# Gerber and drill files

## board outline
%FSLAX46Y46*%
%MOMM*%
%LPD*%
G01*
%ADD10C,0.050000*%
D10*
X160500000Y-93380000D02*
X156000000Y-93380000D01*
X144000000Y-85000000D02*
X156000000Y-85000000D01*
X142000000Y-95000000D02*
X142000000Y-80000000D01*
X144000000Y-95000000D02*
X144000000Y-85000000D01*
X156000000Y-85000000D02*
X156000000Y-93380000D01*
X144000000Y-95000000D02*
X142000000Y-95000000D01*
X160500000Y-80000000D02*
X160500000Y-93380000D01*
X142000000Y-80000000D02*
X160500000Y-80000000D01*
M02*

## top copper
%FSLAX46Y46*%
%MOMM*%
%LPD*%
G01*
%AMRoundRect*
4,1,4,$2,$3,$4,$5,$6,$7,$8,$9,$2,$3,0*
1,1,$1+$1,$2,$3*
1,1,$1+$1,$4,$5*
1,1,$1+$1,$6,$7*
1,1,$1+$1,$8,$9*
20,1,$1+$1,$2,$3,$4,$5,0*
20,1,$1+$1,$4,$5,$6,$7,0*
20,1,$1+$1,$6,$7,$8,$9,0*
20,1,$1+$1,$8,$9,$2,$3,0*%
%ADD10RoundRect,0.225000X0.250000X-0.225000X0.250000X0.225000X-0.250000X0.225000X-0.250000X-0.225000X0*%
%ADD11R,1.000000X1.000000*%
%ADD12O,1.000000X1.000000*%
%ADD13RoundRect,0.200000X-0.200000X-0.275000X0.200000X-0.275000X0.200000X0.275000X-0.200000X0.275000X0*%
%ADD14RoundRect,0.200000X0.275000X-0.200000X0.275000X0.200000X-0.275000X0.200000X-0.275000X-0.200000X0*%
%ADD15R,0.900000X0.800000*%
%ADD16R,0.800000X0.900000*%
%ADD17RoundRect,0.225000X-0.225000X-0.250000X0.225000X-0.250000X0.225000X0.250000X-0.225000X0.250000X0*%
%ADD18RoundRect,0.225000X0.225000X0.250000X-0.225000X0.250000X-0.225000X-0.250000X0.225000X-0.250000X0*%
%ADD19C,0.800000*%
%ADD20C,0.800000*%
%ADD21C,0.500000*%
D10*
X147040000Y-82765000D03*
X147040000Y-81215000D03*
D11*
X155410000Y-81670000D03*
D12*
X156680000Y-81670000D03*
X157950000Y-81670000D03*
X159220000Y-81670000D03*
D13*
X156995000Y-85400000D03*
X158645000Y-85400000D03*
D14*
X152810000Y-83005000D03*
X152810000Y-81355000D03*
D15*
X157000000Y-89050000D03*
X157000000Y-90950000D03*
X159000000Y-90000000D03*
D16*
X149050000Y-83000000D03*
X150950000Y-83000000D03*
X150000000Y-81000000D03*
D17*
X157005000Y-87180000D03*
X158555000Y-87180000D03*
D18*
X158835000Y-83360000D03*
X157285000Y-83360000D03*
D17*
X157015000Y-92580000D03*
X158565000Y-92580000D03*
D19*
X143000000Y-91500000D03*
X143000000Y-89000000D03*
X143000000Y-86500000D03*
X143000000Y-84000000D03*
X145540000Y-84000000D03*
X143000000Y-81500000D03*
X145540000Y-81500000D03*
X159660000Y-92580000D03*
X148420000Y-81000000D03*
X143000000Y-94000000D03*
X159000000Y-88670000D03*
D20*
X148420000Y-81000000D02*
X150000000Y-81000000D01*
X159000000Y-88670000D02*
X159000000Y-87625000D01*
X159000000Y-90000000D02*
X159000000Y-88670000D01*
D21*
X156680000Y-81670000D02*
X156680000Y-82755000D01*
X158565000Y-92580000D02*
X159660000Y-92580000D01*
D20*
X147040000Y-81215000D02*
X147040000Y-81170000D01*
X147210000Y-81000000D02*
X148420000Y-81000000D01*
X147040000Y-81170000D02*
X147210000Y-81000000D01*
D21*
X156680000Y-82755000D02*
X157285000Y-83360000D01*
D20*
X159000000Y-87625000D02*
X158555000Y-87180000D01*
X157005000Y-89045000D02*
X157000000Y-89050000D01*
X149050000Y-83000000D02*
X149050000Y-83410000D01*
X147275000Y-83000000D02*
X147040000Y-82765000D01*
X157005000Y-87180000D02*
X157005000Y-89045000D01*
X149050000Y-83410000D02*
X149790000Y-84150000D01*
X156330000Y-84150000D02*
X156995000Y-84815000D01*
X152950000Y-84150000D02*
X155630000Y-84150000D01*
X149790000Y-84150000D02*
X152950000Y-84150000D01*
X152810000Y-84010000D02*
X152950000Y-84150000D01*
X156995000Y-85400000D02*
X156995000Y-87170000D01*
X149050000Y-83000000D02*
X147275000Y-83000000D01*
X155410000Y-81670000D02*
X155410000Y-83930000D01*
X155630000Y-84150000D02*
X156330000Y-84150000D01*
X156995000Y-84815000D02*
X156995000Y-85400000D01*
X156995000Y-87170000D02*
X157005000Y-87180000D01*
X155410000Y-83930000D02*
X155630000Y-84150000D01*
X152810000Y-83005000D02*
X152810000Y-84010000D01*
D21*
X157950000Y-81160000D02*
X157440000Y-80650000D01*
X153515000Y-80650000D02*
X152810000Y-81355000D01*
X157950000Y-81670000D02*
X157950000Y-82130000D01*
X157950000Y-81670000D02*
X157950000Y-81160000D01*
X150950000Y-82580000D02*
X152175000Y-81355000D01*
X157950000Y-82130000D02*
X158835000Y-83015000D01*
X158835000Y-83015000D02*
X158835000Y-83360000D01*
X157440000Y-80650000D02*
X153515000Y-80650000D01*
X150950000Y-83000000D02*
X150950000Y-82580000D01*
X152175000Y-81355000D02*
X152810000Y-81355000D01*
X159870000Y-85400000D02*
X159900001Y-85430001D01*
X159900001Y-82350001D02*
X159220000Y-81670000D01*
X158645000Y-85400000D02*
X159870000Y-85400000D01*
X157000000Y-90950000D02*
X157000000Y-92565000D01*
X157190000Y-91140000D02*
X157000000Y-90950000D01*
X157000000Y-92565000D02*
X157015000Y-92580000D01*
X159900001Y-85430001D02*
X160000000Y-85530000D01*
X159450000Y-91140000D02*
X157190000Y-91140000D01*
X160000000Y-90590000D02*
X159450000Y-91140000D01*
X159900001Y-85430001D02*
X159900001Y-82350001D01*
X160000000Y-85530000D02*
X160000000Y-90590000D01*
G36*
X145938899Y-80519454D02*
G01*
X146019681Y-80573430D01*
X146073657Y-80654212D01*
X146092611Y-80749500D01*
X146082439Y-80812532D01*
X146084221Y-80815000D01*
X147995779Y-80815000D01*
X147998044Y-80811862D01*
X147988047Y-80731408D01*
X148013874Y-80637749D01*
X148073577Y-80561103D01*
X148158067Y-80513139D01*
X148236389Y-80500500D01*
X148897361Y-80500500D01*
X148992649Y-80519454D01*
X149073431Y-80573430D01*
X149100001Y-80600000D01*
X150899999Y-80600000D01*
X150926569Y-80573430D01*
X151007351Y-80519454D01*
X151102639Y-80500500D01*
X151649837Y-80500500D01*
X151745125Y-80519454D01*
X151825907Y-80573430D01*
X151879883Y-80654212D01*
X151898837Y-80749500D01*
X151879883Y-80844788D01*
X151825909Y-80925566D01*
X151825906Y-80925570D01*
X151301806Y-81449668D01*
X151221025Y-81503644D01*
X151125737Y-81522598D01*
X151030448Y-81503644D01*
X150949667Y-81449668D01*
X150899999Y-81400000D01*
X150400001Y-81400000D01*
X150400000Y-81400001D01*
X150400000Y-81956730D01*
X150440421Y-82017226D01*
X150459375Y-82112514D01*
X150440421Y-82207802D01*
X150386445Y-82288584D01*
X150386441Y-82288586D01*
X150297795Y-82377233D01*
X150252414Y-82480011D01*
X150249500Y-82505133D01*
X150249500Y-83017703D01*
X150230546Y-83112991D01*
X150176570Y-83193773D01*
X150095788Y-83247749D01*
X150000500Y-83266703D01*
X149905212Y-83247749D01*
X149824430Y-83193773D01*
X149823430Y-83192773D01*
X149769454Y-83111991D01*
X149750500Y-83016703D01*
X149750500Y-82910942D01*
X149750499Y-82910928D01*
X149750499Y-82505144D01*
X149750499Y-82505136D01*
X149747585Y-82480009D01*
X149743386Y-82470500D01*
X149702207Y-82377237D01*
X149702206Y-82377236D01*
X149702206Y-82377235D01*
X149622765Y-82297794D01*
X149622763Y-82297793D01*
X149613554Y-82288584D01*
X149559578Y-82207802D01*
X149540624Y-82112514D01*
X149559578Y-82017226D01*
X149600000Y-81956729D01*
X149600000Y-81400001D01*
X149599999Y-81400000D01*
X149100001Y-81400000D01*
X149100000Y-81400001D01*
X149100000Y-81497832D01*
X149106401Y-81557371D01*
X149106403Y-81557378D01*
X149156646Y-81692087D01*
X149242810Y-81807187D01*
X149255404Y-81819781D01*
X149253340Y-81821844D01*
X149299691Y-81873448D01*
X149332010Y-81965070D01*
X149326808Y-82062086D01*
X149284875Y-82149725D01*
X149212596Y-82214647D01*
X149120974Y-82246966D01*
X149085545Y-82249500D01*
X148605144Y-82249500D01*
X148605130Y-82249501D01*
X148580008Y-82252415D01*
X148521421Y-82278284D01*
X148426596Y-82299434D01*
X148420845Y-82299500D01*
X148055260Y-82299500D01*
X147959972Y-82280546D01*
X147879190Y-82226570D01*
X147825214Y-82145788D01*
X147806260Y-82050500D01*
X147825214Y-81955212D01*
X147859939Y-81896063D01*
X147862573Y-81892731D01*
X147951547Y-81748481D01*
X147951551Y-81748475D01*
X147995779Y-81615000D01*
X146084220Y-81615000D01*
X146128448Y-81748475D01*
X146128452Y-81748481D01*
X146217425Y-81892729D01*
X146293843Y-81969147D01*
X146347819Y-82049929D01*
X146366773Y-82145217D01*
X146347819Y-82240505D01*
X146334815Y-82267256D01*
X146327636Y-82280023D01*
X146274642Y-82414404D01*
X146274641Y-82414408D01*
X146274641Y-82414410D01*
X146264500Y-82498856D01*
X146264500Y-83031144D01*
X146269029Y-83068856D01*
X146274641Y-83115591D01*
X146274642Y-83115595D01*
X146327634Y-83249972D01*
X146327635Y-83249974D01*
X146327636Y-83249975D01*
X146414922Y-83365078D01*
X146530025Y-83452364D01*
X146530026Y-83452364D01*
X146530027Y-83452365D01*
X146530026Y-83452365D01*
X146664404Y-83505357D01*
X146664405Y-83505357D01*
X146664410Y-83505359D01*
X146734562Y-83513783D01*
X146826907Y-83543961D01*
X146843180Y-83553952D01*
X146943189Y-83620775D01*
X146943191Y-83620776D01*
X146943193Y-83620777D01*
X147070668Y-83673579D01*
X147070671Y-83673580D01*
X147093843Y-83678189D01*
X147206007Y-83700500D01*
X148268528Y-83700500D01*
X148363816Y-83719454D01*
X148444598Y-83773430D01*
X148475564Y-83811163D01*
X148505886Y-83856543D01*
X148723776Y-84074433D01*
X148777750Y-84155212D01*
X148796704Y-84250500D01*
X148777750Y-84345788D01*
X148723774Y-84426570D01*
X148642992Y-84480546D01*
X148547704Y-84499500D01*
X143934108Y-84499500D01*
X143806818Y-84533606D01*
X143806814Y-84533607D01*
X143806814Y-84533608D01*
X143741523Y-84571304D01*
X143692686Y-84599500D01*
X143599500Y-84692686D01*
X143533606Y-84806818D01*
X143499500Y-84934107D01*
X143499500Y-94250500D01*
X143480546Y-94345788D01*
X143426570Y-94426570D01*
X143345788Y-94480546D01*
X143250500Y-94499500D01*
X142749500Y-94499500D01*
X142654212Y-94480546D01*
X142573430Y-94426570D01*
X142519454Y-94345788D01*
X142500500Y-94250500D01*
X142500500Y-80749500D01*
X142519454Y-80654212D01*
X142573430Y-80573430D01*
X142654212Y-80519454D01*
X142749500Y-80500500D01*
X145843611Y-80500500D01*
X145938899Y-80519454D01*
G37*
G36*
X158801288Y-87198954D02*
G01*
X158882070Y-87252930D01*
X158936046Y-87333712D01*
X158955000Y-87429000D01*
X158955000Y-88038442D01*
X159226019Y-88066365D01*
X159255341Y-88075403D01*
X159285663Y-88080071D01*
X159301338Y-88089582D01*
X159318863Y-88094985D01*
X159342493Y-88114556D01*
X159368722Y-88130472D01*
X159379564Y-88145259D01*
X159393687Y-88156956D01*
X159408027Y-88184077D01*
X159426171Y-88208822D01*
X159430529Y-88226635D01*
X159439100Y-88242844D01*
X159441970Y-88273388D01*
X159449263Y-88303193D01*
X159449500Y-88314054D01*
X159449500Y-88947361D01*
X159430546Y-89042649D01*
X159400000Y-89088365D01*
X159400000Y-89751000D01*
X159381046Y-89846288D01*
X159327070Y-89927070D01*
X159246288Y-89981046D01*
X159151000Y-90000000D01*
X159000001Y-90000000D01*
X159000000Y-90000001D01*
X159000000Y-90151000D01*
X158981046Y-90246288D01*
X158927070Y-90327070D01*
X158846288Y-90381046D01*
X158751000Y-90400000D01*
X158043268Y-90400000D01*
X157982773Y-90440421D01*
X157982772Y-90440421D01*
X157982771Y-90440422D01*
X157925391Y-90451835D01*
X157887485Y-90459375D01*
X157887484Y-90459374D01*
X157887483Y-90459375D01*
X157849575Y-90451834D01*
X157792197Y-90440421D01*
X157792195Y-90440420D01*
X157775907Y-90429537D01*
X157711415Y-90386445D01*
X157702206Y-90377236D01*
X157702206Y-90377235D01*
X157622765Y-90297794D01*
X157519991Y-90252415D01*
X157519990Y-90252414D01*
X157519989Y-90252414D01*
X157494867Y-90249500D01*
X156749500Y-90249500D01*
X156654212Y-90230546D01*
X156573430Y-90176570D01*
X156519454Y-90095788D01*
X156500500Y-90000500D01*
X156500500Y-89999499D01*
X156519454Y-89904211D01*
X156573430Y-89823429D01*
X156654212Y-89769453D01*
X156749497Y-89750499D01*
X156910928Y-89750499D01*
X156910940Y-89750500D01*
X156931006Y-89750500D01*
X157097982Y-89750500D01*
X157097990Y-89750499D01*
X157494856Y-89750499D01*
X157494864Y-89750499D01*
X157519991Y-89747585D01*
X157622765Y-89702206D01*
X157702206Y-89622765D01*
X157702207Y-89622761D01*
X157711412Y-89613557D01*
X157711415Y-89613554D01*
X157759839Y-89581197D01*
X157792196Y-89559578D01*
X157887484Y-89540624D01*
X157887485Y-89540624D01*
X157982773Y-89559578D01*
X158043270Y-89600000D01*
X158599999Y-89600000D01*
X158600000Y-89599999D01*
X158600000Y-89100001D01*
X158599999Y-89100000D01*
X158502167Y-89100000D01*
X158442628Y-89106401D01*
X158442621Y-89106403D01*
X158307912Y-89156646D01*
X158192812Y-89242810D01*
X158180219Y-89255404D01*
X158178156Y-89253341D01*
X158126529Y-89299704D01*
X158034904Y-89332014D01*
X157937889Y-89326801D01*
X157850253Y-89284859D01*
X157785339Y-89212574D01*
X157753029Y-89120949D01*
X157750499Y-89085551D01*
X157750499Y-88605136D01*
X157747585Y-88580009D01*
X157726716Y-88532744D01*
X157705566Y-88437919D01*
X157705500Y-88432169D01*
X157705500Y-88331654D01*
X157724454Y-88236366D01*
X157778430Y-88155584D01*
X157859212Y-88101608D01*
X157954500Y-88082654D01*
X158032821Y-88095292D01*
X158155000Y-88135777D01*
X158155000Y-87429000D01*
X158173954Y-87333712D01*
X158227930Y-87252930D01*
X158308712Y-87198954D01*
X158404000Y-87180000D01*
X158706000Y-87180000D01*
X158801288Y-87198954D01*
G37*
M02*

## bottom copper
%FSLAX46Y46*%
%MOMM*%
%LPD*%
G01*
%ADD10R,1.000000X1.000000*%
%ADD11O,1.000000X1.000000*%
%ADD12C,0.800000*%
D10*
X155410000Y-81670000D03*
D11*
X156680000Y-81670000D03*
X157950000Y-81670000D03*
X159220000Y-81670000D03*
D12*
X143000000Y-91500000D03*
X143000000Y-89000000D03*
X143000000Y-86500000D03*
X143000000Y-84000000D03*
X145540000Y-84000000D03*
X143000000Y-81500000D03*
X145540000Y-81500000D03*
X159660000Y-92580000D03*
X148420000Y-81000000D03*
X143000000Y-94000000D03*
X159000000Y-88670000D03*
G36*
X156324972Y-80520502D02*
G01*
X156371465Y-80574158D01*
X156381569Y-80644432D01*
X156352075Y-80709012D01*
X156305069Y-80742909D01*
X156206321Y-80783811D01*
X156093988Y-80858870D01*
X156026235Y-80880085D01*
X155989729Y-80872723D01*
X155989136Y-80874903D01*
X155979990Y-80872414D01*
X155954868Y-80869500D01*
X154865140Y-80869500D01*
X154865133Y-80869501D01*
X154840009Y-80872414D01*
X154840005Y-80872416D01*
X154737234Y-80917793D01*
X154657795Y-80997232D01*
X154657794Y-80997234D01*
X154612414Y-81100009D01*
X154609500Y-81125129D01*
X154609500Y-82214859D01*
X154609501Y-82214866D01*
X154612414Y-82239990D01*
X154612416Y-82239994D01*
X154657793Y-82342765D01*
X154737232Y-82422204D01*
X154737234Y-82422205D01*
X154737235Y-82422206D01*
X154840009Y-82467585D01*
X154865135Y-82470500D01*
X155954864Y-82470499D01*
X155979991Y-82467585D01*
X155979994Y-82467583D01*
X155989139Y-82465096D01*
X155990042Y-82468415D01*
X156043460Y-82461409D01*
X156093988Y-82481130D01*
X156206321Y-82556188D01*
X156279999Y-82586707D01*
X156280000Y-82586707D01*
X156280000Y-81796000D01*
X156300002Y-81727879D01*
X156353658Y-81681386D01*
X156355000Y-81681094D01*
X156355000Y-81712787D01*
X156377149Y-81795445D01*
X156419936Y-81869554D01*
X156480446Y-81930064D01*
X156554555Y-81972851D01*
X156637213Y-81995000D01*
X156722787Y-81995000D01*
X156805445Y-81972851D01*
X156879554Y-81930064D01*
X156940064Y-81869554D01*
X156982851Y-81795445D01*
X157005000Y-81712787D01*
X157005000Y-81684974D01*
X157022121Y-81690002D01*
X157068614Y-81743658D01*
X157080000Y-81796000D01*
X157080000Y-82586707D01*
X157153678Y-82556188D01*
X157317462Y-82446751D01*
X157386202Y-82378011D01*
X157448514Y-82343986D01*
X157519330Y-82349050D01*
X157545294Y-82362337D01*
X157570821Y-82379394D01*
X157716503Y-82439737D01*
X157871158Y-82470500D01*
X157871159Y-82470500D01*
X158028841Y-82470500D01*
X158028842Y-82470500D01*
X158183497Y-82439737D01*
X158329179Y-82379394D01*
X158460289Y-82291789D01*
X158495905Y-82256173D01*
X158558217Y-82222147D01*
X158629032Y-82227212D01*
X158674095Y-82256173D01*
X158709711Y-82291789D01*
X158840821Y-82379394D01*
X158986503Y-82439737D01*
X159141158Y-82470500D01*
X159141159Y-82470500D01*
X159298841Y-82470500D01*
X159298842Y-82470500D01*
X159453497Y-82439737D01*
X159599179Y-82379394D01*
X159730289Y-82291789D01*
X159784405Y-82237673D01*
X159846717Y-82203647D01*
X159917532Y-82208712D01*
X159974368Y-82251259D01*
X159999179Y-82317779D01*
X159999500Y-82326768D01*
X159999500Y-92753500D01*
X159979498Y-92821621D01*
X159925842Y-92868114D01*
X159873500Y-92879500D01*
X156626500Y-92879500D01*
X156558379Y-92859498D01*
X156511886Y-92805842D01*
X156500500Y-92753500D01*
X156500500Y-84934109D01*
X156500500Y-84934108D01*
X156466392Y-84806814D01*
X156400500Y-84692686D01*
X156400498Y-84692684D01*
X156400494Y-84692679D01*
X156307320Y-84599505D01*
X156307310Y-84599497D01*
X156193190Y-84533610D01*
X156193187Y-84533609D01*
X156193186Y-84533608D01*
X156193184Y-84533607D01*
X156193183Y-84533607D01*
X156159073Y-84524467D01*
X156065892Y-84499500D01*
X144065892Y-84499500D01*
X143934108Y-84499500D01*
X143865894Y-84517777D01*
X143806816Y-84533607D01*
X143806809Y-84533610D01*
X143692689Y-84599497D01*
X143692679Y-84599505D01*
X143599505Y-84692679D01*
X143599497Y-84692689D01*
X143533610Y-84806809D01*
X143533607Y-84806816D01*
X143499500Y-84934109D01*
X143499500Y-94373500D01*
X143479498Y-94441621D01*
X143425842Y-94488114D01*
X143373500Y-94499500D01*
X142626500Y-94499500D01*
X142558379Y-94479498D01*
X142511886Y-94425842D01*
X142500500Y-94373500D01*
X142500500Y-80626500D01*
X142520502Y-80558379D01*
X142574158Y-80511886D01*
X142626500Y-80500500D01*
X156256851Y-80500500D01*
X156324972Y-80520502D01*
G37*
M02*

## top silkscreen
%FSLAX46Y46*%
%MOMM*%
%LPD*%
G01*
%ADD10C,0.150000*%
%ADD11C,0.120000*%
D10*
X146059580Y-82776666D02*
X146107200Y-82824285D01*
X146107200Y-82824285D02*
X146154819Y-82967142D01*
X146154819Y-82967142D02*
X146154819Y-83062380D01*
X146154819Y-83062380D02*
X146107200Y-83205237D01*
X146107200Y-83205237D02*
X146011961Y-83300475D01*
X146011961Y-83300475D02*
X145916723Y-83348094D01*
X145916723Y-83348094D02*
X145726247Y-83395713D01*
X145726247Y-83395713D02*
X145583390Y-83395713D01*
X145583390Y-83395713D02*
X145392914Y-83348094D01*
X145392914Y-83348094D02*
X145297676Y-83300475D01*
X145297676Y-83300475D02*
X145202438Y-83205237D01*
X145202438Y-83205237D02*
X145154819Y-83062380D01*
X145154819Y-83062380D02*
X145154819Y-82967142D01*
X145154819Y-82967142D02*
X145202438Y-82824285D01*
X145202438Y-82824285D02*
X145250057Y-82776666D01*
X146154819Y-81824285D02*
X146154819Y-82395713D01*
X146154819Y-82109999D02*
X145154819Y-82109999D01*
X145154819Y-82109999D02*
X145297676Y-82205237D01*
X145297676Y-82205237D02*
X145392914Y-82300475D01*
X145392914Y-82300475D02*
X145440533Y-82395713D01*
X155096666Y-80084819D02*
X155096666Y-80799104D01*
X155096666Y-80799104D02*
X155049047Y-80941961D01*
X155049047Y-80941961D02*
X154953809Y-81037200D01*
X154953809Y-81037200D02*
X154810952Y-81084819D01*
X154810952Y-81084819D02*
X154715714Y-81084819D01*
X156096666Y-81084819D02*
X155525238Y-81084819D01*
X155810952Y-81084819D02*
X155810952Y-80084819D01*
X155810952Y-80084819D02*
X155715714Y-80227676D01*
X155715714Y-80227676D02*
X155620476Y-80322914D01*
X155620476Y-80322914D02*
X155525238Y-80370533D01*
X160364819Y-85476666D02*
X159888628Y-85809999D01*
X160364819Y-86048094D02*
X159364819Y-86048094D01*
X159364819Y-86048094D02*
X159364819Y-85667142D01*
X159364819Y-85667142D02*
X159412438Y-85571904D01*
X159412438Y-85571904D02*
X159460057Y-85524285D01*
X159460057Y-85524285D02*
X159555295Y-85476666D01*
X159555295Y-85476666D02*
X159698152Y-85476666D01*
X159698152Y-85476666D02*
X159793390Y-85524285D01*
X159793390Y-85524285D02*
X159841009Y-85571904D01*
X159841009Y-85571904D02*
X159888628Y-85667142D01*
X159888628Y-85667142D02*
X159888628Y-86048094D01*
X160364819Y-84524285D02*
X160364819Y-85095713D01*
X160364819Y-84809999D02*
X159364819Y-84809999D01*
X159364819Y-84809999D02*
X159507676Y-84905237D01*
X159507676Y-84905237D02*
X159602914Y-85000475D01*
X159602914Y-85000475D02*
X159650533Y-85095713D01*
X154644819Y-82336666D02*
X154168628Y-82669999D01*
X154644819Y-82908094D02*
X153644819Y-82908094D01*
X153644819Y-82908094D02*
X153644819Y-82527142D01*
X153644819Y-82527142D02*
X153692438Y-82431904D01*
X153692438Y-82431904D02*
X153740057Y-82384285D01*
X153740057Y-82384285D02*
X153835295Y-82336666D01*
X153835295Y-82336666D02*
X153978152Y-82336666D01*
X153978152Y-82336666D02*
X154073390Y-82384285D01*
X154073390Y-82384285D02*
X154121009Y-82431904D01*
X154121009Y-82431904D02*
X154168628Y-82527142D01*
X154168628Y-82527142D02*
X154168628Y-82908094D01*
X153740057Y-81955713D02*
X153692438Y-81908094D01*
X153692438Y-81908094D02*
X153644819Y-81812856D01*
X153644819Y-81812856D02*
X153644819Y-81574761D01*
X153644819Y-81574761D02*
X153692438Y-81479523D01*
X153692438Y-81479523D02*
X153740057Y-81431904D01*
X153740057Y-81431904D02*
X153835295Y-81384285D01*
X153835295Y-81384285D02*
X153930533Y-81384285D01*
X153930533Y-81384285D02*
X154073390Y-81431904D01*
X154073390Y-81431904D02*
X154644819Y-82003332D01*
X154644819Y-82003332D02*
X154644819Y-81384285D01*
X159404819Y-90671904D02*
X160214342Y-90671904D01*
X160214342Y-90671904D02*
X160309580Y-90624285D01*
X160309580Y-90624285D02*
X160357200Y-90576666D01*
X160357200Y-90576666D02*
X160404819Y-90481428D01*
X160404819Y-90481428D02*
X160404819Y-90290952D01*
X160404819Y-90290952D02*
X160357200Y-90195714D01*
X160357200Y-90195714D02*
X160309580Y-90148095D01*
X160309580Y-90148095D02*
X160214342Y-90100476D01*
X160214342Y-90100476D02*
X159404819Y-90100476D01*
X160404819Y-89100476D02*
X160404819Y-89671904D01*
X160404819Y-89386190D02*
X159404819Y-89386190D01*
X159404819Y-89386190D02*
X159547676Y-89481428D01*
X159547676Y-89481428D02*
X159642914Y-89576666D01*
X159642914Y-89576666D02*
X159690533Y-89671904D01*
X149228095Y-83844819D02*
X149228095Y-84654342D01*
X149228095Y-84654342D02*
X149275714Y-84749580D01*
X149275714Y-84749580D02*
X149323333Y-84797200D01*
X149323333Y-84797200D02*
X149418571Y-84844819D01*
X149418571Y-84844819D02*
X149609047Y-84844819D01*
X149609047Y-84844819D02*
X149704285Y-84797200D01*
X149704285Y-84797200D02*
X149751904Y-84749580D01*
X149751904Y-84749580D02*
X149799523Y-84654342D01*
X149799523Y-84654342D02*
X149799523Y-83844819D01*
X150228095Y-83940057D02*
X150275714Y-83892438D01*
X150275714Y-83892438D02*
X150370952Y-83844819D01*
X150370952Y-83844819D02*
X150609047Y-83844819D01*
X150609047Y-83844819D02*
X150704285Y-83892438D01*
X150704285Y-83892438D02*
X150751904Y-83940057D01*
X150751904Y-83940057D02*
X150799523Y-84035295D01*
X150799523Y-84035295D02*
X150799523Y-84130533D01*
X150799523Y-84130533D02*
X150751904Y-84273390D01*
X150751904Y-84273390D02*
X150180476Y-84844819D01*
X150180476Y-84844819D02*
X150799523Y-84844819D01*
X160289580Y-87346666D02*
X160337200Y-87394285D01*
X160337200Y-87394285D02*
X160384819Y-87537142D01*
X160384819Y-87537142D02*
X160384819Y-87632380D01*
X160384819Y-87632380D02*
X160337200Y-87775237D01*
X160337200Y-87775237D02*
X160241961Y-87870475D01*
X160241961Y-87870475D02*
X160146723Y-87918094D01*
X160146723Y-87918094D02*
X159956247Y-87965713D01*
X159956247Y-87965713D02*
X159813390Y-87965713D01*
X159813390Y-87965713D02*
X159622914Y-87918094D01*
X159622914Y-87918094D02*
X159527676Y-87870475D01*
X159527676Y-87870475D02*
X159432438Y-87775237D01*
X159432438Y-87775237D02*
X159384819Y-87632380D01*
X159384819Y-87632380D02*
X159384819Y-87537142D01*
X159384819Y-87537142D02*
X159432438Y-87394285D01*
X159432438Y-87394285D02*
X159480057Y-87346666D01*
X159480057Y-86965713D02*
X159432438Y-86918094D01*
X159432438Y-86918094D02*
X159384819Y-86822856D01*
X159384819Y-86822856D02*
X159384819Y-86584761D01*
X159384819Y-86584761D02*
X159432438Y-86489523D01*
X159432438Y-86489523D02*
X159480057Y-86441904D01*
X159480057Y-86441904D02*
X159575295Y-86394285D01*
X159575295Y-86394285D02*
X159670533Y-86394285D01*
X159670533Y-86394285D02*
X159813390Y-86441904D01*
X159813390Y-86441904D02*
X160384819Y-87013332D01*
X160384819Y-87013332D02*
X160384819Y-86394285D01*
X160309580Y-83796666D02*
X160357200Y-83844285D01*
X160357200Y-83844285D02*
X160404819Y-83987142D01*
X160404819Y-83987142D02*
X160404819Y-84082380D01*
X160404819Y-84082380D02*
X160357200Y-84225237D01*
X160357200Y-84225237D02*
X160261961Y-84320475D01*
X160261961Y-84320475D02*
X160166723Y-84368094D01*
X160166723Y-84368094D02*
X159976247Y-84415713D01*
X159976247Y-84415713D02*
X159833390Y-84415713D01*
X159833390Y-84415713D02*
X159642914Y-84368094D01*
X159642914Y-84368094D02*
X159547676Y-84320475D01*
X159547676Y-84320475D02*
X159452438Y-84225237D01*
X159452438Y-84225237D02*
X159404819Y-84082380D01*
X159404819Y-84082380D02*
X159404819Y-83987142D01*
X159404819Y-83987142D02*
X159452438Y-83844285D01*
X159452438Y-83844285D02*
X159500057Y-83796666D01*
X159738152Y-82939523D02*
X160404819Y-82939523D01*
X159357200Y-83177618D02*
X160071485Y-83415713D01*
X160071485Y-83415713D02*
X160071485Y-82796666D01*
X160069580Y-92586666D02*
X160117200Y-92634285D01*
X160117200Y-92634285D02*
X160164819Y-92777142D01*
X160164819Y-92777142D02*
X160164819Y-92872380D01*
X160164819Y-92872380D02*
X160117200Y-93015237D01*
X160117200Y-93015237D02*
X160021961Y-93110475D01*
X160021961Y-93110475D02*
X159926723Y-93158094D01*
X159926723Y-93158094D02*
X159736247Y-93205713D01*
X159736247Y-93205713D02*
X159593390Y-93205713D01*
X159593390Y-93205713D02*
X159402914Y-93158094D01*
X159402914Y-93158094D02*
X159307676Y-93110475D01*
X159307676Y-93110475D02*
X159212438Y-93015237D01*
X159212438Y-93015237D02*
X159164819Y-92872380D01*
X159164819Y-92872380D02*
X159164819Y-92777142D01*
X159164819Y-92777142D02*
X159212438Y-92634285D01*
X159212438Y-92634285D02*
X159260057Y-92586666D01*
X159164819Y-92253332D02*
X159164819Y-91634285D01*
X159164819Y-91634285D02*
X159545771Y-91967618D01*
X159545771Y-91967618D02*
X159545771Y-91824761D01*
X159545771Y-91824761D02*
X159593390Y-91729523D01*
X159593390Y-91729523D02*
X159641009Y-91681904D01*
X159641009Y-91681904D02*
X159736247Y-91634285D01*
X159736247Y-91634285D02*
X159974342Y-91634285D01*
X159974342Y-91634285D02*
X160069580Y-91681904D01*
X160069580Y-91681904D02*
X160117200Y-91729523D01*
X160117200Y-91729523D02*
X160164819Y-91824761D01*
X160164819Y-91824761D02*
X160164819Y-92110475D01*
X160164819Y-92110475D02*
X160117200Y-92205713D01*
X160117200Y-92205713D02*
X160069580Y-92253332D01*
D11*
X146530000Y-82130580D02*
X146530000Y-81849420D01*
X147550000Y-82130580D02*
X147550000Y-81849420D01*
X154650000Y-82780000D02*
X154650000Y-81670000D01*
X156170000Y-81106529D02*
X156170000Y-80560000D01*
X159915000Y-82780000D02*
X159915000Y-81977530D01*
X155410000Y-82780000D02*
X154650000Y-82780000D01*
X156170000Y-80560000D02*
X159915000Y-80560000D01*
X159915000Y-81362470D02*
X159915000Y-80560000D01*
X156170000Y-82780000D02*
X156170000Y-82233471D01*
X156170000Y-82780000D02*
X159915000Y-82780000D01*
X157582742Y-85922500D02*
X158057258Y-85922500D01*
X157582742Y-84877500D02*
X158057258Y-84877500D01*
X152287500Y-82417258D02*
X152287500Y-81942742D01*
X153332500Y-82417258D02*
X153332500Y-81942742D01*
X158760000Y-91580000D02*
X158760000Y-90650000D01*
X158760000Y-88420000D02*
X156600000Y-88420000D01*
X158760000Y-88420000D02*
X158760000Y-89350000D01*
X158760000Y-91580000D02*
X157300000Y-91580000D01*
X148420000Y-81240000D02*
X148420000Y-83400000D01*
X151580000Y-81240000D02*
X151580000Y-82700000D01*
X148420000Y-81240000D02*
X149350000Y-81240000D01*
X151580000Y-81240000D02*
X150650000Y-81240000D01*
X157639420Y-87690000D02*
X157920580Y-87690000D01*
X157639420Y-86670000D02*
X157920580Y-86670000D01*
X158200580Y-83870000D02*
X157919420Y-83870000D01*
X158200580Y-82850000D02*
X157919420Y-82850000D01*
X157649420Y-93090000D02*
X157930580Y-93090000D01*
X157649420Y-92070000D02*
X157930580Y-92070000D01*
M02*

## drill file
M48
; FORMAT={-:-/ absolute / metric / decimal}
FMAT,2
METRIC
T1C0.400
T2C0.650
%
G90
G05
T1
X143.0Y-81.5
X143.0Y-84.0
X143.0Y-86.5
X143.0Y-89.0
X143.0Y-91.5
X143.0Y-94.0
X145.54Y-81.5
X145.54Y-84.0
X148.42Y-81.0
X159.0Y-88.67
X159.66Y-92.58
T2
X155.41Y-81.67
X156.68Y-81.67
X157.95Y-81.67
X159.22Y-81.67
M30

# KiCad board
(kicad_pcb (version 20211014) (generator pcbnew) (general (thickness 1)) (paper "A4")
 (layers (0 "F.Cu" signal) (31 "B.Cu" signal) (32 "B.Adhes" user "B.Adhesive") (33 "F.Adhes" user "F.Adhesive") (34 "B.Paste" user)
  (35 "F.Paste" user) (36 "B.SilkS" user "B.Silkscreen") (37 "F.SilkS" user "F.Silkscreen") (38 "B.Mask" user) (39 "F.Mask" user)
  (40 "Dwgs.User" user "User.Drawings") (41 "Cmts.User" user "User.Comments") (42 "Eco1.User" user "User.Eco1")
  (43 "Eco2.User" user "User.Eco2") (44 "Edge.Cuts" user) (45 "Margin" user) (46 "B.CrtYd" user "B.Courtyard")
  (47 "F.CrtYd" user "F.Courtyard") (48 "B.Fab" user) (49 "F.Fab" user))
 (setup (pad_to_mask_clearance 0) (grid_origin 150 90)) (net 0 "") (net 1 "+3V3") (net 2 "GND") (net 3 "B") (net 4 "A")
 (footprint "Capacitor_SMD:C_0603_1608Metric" (layer "F.Cu") (at 147.04 81.99 90)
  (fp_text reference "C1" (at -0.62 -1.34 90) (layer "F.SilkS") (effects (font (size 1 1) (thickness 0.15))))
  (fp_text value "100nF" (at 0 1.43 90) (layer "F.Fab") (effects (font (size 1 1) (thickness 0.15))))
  (fp_line (start -0.14058 -0.51) (end 0.14058 -0.51) (layer "F.SilkS") (width 0.12))
  (fp_line (start -0.14058 0.51) (end 0.14058 0.51) (layer "F.SilkS") (width 0.12))
  (pad "1" smd roundrect locked (at -0.775 0 90) (size 0.9 0.95) (layers "F.Cu" "F.Paste" "F.Mask") (roundrect_rratio 0.25) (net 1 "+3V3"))
  (pad "2" smd roundrect locked (at 0.775 0 90) (size 0.9 0.95) (layers "F.Cu" "F.Paste" "F.Mask") (roundrect_rratio 0.25) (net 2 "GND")))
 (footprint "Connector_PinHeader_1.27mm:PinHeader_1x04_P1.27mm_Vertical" (layer "F.Cu") (at 155.41 81.67 90)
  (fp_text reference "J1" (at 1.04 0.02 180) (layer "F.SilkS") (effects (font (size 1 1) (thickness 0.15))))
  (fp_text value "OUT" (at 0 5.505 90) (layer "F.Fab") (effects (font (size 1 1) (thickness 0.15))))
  (fp_line (start -1.11 -0.76) (end 0 -0.76) (layer "F.SilkS") (width 0.12))
  (fp_line (start 0.563471 0.76) (end 1.11 0.76) (layer "F.SilkS") (width 0.12))
  (fp_line (start -1.11 4.505) (end -0.30753 4.505) (layer "F.SilkS") (width 0.12))
  (fp_line (start -1.11 0) (end -1.11 -0.76) (layer "F.SilkS") (width 0.12))
  (fp_line (start 1.11 0.76) (end 1.11 4.505) (layer "F.SilkS") (width 0.12))
  (fp_line (start 0.30753 4.505) (end 1.11 4.505) (layer "F.SilkS") (width 0.12))
  (fp_line (start -1.11 0.76) (end -0.563471 0.76) (layer "F.SilkS") (width 0.12))
  (fp_line (start -1.11 0.76) (end -1.11 4.505) (layer "F.SilkS") (width 0.12))
  (pad "1" thru_hole rect locked (at 0 0 90) (size 1 1) (drill 0.65) (layers *.Cu *.Mask) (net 1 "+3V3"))
  (pad "2" thru_hole oval locked (at 0 1.27 90) (size 1 1) (drill 0.65) (layers *.Cu *.Mask) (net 2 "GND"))
  (pad "3" thru_hole oval locked (at 0 2.54 90) (size 1 1) (drill 0.65) (layers *.Cu *.Mask) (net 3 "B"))
  (pad "4" thru_hole oval locked (at 0 3.81 90) (size 1 1) (drill 0.65) (layers *.Cu *.Mask) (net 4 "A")))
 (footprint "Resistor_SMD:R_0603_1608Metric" (layer "F.Cu") (at 157.82 85.4)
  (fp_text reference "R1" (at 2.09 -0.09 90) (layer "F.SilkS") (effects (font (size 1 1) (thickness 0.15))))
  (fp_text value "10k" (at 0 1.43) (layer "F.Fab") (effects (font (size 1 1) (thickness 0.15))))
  (fp_line (start -0.237258 0.5225) (end 0.237258 0.5225) (layer "F.SilkS") (width 0.12))
  (fp_line (start -0.237258 -0.5225) (end 0.237258 -0.5225) (layer "F.SilkS") (width 0.12))
  (pad "1" smd roundrect locked (at -0.825 0) (size 0.8 0.95) (layers "F.Cu" "F.Paste" "F.Mask") (roundrect_rratio 0.25) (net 1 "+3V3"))
  (pad "2" smd roundrect locked (at 0.825 0) (size 0.8 0.95) (layers "F.Cu" "F.Paste" "F.Mask") (roundrect_rratio 0.25) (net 4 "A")))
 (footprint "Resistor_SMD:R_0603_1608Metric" (layer "F.Cu") (at 152.81 82.18 90)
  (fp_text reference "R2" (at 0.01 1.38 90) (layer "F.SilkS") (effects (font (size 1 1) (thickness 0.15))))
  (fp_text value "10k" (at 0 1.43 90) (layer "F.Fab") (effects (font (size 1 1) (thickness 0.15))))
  (fp_line (start -0.237258 -0.5225) (end 0.237258 -0.5225) (layer "F.SilkS") (width 0.12))
  (fp_line (start -0.237258 0.5225) (end 0.237258 0.5225) (layer "F.SilkS") (width 0.12))
  (pad "1" smd roundrect locked (at -0.825 0 90) (size 0.8 0.95) (layers "F.Cu" "F.Paste" "F.Mask") (roundrect_rratio 0.25) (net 1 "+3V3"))
  (pad "2" smd roundrect locked (at 0.825 0 90) (size 0.8 0.95) (layers "F.Cu" "F.Paste" "F.Mask") (roundrect_rratio 0.25) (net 3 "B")))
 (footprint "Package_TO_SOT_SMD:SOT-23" (layer "F.Cu") (at 158 90)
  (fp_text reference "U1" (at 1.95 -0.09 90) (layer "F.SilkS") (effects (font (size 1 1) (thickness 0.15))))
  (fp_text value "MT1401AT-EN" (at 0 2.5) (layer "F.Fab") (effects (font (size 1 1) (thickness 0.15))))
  (fp_line (start 0.76 1.58) (end 0.76 0.65) (layer "F.SilkS") (width 0.12))
  (fp_line (start 0.76 -1.58) (end -1.4 -1.58) (layer "F.SilkS") (width 0.12))
  (fp_line (start 0.76 -1.58) (end 0.76 -0.65) (layer "F.SilkS") (width 0.12))
  (fp_line (start 0.76 1.58) (end -0.7 1.58) (layer "F.SilkS") (width 0.12))
  (pad "1" smd rect locked (at -1 -0.95) (size 0.9 0.8) (layers "F.Cu" "F.Paste" "F.Mask") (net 1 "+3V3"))
  (pad "2" smd rect locked (at -1 0.95) (size 0.9 0.8) (layers "F.Cu" "F.Paste" "F.Mask") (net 4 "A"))
  (pad "3" smd rect locked (at 1 0) (size 0.9 0.8) (layers "F.Cu" "F.Paste" "F.Mask") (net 2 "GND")))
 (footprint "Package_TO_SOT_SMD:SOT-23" (layer "F.Cu") (at 150 82 90)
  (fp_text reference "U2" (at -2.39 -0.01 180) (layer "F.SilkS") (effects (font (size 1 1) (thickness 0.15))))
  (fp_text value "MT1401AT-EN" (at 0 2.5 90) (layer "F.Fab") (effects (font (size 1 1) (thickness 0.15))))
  (fp_line (start 0.76 -1.58) (end -1.4 -1.58) (layer "F.SilkS") (width 0.12))
  (fp_line (start 0.76 1.58) (end -0.7 1.58) (layer "F.SilkS") (width 0.12))
  (fp_line (start 0.76 -1.58) (end 0.76 -0.65) (layer "F.SilkS") (width 0.12))
  (fp_line (start 0.76 1.58) (end 0.76 0.65) (layer "F.SilkS") (width 0.12))
  (pad "1" smd rect locked (at -1 -0.95 90) (size 0.9 0.8) (layers "F.Cu" "F.Paste" "F.Mask") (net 1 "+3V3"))
  (pad "2" smd rect locked (at -1 0.95 90) (size 0.9 0.8) (layers "F.Cu" "F.Paste" "F.Mask") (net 3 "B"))
  (pad "3" smd rect locked (at 1 0 90) (size 0.9 0.8) (layers "F.Cu" "F.Paste" "F.Mask") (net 2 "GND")))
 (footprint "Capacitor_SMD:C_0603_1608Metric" (layer "F.Cu") (at 157.78 87.18)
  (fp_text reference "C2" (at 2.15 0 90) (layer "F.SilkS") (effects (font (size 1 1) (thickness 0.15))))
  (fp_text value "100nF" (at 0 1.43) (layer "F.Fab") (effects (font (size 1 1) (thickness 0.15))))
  (fp_line (start -0.14058 0.51) (end 0.14058 0.51) (layer "F.SilkS") (width 0.12))
  (fp_line (start -0.14058 -0.51) (end 0.14058 -0.51) (layer "F.SilkS") (width 0.12))
  (pad "1" smd roundrect locked (at -0.775 0) (size 0.9 0.95) (layers "F.Cu" "F.Paste" "F.Mask") (roundrect_rratio 0.25) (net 1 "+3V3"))
  (pad "2" smd roundrect locked (at 0.775 0) (size 0.9 0.95) (layers "F.Cu" "F.Paste" "F.Mask") (roundrect_rratio 0.25) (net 2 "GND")))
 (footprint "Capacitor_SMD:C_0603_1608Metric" (layer "F.Cu") (at 158.06 83.36 180)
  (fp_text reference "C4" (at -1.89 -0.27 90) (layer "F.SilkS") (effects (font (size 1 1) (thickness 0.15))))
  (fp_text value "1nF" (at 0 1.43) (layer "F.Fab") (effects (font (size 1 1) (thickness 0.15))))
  (fp_line (start -0.14058 -0.51) (end 0.14058 -0.51) (layer "F.SilkS") (width 0.12))
  (fp_line (start -0.14058 0.51) (end 0.14058 0.51) (layer "F.SilkS") (width 0.12))
  (pad "1" smd roundrect (at -0.775 0 180) (size 0.9 0.95) (layers "F.Cu" "F.Paste" "F.Mask") (roundrect_rratio 0.25) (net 3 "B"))
  (pad "2" smd roundrect (at 0.775 0 180) (size 0.9 0.95) (layers "F.Cu" "F.Paste" "F.Mask") (roundrect_rratio 0.25) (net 2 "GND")))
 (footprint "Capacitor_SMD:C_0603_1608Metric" (layer "F.Cu") (at 157.79 92.58)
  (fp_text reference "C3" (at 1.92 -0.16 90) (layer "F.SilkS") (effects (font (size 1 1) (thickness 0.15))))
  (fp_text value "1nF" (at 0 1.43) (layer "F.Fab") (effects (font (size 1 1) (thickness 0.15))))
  (fp_line (start -0.14058 0.51) (end 0.14058 0.51) (layer "F.SilkS") (width 0.12))
  (fp_line (start -0.14058 -0.51) (end 0.14058 -0.51) (layer "F.SilkS") (width 0.12))
  (pad "1" smd roundrect (at -0.775 0) (size 0.9 0.95) (layers "F.Cu" "F.Paste" "F.Mask") (roundrect_rratio 0.25) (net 4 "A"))
  (pad "2" smd roundrect (at 0.775 0) (size 0.9 0.95) (layers "F.Cu" "F.Paste" "F.Mask") (roundrect_rratio 0.25) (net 2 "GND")))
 (gr_line (start 160.5 93.38) (end 156 93.38) (layer "Edge.Cuts") (width 0.05))
 (gr_line (start 144 85) (end 156 85) (layer "Edge.Cuts") (width 0.05))
 (gr_line (start 142 95) (end 142 80) (layer "Edge.Cuts") (width 0.05))
 (gr_line (start 144 95) (end 144 85) (layer "Edge.Cuts") (width 0.05))
 (gr_line (start 156 85) (end 156 93.38) (layer "Edge.Cuts") (width 0.05))
 (gr_line (start 144 95) (end 142 95) (layer "Edge.Cuts") (width 0.05))
 (gr_line (start 160.5 80) (end 160.5 93.38) (layer "Edge.Cuts") (width 0.05))
 (gr_line (start 142 80) (end 160.5 80) (layer "Edge.Cuts") (width 0.05))
 (segment (start 148.42 81) (end 150 81) (width 0.8) (layer "F.Cu") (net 2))
 (segment (start 159 88.67) (end 159 87.625) (width 0.8) (layer "F.Cu") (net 2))
 (segment (start 159 90) (end 159 88.67) (width 0.8) (layer "F.Cu") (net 2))
 (segment (start 156.68 81.67) (end 156.68 82.755) (width 0.5) (layer "F.Cu") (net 2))
 (segment (start 158.565 92.58) (end 159.66 92.58) (width 0.5) (layer "F.Cu") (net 2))
 (segment (start 147.04 81.215) (end 147.04 81.17) (width 0.8) (layer "F.Cu") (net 2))
 (segment (start 147.21 81) (end 148.42 81) (width 0.8) (layer "F.Cu") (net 2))
 (segment (start 147.04 81.17) (end 147.21 81) (width 0.8) (layer "F.Cu") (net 2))
 (segment (start 156.68 82.755) (end 157.285 83.36) (width 0.5) (layer "F.Cu") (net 2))
 (segment (start 159 87.625) (end 158.555 87.18) (width 0.8) (layer "F.Cu") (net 2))
 (via (at 143 91.5) (size 0.8) (drill 0.4) (layers "F.Cu" "B.Cu") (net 2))
 (via (at 143 89) (size 0.8) (drill 0.4) (layers "F.Cu" "B.Cu") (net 2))
 (via (at 143 86.5) (size 0.8) (drill 0.4) (layers "F.Cu" "B.Cu") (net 2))
 (via (at 143 84) (size 0.8) (drill 0.4) (layers "F.Cu" "B.Cu") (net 2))
 (via (at 145.54 84) (size 0.8) (drill 0.4) (layers "F.Cu" "B.Cu") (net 2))
 (via (at 143 81.5) (size 0.8) (drill 0.4) (layers "F.Cu" "B.Cu") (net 2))
 (via (at 145.54 81.5) (size 0.8) (drill 0.4) (layers "F.Cu" "B.Cu") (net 2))
 (via (at 159.66 92.58) (size 0.8) (drill 0.4) (layers "F.Cu" "B.Cu") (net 2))
 (via (at 148.42 81) (size 0.8) (drill 0.4) (layers "F.Cu" "B.Cu") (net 2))
 (via (at 143 94) (size 0.8) (drill 0.4) (layers "F.Cu" "B.Cu") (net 2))
 (via (at 159 88.67) (size 0.8) (drill 0.4) (layers "F.Cu" "B.Cu") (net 2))
 (segment (start 157.005 89.045) (end 157 89.05) (width 0.8) (layer "F.Cu") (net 1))
 (segment (start 149.05 83) (end 149.05 83.41) (width 0.8) (layer "F.Cu") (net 1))
 (segment (start 147.275 83) (end 147.04 82.765) (width 0.8) (layer "F.Cu") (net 1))
 (segment (start 157.005 87.18) (end 157.005 89.045) (width 0.8) (layer "F.Cu") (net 1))
 (segment (start 149.05 83.41) (end 149.79 84.15) (width 0.8) (layer "F.Cu") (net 1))
 (segment (start 156.33 84.15) (end 156.995 84.815) (width 0.8) (layer "F.Cu") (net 1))
 (segment (start 152.95 84.15) (end 155.63 84.15) (width 0.8) (layer "F.Cu") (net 1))
 (segment (start 149.79 84.15) (end 152.95 84.15) (width 0.8) (layer "F.Cu") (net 1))
 (segment (start 152.81 84.01) (end 152.95 84.15) (width 0.8) (layer "F.Cu") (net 1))
 (segment (start 156.995 85.4) (end 156.995 87.17) (width 0.8) (layer "F.Cu") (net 1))
 (segment (start 149.05 83) (end 147.275 83) (width 0.8) (layer "F.Cu") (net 1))
 (segment (start 155.41 81.67) (end 155.41 83.93) (width 0.8) (layer "F.Cu") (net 1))
 (segment (start 155.63 84.15) (end 156.33 84.15) (width 0.8) (layer "F.Cu") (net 1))
 (segment (start 156.995 84.815) (end 156.995 85.4) (width 0.8) (layer "F.Cu") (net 1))
 (segment (start 156.995 87.17) (end 157.005 87.18) (width 0.8) (layer "F.Cu") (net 1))
 (segment (start 155.41 83.93) (end 155.63 84.15) (width 0.8) (layer "F.Cu") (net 1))
 (segment (start 152.81 83.005) (end 152.81 84.01) (width 0.8) (layer "F.Cu") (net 1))
 (segment (start 157.95 81.16) (end 157.44 80.65) (width 0.5) (layer "F.Cu") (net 3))
 (segment (start 153.515 80.65) (end 152.81 81.355) (width 0.5) (layer "F.Cu") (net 3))
 (segment (start 157.95 81.67) (end 157.95 82.13) (width 0.5) (layer "F.Cu") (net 3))
 (segment (start 157.95 81.67) (end 157.95 81.16) (width 0.5) (layer "F.Cu") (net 3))
 (segment (start 150.95 82.58) (end 152.175 81.355) (width 0.5) (layer "F.Cu") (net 3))
 (segment (start 157.95 82.13) (end 158.835 83.015) (width 0.5) (layer "F.Cu") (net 3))
 (segment (start 158.835 83.015) (end 158.835 83.36) (width 0.5) (layer "F.Cu") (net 3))
 (segment (start 157.44 80.65) (end 153.515 80.65) (width 0.5) (layer "F.Cu") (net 3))
 (segment (start 150.95 83) (end 150.95 82.58) (width 0.5) (layer "F.Cu") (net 3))
 (segment (start 152.175 81.355) (end 152.81 81.355) (width 0.5) (layer "F.Cu") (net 3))
 (segment (start 159.87 85.4) (end 159.900001 85.430001) (width 0.5) (layer "F.Cu") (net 4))
 (segment (start 159.900001 82.350001) (end 159.22 81.67) (width 0.5) (layer "F.Cu") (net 4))
 (segment (start 158.645 85.4) (end 159.87 85.4) (width 0.5) (layer "F.Cu") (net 4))
 (segment (start 157 90.95) (end 157 92.565) (width 0.5) (layer "F.Cu") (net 4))
 (segment (start 157.19 91.14) (end 157 90.95) (width 0.5) (layer "F.Cu") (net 4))
 (segment (start 157 92.565) (end 157.015 92.58) (width 0.5) (layer "F.Cu") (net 4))
 (segment (start 159.900001 85.430001) (end 160 85.53) (width 0.5) (layer "F.Cu") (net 4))
 (segment (start 159.45 91.14) (end 157.19 91.14) (width 0.5) (layer "F.Cu") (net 4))
 (segment (start 160 90.59) (end 159.45 91.14) (width 0.5) (layer "F.Cu") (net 4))
 (segment (start 159.900001 85.430001) (end 159.900001 82.350001) (width 0.5) (layer "F.Cu") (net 4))
 (segment (start 160 85.53) (end 160 90.59) (width 0.5) (layer "F.Cu") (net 4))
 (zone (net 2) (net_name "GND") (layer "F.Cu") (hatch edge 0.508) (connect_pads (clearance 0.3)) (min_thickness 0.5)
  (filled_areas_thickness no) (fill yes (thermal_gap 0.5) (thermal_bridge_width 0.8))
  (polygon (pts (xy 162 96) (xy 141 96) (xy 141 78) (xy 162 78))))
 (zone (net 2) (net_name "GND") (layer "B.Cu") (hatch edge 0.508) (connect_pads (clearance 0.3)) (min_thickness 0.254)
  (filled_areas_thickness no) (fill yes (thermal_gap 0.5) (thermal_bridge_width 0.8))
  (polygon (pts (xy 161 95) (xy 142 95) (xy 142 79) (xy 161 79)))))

